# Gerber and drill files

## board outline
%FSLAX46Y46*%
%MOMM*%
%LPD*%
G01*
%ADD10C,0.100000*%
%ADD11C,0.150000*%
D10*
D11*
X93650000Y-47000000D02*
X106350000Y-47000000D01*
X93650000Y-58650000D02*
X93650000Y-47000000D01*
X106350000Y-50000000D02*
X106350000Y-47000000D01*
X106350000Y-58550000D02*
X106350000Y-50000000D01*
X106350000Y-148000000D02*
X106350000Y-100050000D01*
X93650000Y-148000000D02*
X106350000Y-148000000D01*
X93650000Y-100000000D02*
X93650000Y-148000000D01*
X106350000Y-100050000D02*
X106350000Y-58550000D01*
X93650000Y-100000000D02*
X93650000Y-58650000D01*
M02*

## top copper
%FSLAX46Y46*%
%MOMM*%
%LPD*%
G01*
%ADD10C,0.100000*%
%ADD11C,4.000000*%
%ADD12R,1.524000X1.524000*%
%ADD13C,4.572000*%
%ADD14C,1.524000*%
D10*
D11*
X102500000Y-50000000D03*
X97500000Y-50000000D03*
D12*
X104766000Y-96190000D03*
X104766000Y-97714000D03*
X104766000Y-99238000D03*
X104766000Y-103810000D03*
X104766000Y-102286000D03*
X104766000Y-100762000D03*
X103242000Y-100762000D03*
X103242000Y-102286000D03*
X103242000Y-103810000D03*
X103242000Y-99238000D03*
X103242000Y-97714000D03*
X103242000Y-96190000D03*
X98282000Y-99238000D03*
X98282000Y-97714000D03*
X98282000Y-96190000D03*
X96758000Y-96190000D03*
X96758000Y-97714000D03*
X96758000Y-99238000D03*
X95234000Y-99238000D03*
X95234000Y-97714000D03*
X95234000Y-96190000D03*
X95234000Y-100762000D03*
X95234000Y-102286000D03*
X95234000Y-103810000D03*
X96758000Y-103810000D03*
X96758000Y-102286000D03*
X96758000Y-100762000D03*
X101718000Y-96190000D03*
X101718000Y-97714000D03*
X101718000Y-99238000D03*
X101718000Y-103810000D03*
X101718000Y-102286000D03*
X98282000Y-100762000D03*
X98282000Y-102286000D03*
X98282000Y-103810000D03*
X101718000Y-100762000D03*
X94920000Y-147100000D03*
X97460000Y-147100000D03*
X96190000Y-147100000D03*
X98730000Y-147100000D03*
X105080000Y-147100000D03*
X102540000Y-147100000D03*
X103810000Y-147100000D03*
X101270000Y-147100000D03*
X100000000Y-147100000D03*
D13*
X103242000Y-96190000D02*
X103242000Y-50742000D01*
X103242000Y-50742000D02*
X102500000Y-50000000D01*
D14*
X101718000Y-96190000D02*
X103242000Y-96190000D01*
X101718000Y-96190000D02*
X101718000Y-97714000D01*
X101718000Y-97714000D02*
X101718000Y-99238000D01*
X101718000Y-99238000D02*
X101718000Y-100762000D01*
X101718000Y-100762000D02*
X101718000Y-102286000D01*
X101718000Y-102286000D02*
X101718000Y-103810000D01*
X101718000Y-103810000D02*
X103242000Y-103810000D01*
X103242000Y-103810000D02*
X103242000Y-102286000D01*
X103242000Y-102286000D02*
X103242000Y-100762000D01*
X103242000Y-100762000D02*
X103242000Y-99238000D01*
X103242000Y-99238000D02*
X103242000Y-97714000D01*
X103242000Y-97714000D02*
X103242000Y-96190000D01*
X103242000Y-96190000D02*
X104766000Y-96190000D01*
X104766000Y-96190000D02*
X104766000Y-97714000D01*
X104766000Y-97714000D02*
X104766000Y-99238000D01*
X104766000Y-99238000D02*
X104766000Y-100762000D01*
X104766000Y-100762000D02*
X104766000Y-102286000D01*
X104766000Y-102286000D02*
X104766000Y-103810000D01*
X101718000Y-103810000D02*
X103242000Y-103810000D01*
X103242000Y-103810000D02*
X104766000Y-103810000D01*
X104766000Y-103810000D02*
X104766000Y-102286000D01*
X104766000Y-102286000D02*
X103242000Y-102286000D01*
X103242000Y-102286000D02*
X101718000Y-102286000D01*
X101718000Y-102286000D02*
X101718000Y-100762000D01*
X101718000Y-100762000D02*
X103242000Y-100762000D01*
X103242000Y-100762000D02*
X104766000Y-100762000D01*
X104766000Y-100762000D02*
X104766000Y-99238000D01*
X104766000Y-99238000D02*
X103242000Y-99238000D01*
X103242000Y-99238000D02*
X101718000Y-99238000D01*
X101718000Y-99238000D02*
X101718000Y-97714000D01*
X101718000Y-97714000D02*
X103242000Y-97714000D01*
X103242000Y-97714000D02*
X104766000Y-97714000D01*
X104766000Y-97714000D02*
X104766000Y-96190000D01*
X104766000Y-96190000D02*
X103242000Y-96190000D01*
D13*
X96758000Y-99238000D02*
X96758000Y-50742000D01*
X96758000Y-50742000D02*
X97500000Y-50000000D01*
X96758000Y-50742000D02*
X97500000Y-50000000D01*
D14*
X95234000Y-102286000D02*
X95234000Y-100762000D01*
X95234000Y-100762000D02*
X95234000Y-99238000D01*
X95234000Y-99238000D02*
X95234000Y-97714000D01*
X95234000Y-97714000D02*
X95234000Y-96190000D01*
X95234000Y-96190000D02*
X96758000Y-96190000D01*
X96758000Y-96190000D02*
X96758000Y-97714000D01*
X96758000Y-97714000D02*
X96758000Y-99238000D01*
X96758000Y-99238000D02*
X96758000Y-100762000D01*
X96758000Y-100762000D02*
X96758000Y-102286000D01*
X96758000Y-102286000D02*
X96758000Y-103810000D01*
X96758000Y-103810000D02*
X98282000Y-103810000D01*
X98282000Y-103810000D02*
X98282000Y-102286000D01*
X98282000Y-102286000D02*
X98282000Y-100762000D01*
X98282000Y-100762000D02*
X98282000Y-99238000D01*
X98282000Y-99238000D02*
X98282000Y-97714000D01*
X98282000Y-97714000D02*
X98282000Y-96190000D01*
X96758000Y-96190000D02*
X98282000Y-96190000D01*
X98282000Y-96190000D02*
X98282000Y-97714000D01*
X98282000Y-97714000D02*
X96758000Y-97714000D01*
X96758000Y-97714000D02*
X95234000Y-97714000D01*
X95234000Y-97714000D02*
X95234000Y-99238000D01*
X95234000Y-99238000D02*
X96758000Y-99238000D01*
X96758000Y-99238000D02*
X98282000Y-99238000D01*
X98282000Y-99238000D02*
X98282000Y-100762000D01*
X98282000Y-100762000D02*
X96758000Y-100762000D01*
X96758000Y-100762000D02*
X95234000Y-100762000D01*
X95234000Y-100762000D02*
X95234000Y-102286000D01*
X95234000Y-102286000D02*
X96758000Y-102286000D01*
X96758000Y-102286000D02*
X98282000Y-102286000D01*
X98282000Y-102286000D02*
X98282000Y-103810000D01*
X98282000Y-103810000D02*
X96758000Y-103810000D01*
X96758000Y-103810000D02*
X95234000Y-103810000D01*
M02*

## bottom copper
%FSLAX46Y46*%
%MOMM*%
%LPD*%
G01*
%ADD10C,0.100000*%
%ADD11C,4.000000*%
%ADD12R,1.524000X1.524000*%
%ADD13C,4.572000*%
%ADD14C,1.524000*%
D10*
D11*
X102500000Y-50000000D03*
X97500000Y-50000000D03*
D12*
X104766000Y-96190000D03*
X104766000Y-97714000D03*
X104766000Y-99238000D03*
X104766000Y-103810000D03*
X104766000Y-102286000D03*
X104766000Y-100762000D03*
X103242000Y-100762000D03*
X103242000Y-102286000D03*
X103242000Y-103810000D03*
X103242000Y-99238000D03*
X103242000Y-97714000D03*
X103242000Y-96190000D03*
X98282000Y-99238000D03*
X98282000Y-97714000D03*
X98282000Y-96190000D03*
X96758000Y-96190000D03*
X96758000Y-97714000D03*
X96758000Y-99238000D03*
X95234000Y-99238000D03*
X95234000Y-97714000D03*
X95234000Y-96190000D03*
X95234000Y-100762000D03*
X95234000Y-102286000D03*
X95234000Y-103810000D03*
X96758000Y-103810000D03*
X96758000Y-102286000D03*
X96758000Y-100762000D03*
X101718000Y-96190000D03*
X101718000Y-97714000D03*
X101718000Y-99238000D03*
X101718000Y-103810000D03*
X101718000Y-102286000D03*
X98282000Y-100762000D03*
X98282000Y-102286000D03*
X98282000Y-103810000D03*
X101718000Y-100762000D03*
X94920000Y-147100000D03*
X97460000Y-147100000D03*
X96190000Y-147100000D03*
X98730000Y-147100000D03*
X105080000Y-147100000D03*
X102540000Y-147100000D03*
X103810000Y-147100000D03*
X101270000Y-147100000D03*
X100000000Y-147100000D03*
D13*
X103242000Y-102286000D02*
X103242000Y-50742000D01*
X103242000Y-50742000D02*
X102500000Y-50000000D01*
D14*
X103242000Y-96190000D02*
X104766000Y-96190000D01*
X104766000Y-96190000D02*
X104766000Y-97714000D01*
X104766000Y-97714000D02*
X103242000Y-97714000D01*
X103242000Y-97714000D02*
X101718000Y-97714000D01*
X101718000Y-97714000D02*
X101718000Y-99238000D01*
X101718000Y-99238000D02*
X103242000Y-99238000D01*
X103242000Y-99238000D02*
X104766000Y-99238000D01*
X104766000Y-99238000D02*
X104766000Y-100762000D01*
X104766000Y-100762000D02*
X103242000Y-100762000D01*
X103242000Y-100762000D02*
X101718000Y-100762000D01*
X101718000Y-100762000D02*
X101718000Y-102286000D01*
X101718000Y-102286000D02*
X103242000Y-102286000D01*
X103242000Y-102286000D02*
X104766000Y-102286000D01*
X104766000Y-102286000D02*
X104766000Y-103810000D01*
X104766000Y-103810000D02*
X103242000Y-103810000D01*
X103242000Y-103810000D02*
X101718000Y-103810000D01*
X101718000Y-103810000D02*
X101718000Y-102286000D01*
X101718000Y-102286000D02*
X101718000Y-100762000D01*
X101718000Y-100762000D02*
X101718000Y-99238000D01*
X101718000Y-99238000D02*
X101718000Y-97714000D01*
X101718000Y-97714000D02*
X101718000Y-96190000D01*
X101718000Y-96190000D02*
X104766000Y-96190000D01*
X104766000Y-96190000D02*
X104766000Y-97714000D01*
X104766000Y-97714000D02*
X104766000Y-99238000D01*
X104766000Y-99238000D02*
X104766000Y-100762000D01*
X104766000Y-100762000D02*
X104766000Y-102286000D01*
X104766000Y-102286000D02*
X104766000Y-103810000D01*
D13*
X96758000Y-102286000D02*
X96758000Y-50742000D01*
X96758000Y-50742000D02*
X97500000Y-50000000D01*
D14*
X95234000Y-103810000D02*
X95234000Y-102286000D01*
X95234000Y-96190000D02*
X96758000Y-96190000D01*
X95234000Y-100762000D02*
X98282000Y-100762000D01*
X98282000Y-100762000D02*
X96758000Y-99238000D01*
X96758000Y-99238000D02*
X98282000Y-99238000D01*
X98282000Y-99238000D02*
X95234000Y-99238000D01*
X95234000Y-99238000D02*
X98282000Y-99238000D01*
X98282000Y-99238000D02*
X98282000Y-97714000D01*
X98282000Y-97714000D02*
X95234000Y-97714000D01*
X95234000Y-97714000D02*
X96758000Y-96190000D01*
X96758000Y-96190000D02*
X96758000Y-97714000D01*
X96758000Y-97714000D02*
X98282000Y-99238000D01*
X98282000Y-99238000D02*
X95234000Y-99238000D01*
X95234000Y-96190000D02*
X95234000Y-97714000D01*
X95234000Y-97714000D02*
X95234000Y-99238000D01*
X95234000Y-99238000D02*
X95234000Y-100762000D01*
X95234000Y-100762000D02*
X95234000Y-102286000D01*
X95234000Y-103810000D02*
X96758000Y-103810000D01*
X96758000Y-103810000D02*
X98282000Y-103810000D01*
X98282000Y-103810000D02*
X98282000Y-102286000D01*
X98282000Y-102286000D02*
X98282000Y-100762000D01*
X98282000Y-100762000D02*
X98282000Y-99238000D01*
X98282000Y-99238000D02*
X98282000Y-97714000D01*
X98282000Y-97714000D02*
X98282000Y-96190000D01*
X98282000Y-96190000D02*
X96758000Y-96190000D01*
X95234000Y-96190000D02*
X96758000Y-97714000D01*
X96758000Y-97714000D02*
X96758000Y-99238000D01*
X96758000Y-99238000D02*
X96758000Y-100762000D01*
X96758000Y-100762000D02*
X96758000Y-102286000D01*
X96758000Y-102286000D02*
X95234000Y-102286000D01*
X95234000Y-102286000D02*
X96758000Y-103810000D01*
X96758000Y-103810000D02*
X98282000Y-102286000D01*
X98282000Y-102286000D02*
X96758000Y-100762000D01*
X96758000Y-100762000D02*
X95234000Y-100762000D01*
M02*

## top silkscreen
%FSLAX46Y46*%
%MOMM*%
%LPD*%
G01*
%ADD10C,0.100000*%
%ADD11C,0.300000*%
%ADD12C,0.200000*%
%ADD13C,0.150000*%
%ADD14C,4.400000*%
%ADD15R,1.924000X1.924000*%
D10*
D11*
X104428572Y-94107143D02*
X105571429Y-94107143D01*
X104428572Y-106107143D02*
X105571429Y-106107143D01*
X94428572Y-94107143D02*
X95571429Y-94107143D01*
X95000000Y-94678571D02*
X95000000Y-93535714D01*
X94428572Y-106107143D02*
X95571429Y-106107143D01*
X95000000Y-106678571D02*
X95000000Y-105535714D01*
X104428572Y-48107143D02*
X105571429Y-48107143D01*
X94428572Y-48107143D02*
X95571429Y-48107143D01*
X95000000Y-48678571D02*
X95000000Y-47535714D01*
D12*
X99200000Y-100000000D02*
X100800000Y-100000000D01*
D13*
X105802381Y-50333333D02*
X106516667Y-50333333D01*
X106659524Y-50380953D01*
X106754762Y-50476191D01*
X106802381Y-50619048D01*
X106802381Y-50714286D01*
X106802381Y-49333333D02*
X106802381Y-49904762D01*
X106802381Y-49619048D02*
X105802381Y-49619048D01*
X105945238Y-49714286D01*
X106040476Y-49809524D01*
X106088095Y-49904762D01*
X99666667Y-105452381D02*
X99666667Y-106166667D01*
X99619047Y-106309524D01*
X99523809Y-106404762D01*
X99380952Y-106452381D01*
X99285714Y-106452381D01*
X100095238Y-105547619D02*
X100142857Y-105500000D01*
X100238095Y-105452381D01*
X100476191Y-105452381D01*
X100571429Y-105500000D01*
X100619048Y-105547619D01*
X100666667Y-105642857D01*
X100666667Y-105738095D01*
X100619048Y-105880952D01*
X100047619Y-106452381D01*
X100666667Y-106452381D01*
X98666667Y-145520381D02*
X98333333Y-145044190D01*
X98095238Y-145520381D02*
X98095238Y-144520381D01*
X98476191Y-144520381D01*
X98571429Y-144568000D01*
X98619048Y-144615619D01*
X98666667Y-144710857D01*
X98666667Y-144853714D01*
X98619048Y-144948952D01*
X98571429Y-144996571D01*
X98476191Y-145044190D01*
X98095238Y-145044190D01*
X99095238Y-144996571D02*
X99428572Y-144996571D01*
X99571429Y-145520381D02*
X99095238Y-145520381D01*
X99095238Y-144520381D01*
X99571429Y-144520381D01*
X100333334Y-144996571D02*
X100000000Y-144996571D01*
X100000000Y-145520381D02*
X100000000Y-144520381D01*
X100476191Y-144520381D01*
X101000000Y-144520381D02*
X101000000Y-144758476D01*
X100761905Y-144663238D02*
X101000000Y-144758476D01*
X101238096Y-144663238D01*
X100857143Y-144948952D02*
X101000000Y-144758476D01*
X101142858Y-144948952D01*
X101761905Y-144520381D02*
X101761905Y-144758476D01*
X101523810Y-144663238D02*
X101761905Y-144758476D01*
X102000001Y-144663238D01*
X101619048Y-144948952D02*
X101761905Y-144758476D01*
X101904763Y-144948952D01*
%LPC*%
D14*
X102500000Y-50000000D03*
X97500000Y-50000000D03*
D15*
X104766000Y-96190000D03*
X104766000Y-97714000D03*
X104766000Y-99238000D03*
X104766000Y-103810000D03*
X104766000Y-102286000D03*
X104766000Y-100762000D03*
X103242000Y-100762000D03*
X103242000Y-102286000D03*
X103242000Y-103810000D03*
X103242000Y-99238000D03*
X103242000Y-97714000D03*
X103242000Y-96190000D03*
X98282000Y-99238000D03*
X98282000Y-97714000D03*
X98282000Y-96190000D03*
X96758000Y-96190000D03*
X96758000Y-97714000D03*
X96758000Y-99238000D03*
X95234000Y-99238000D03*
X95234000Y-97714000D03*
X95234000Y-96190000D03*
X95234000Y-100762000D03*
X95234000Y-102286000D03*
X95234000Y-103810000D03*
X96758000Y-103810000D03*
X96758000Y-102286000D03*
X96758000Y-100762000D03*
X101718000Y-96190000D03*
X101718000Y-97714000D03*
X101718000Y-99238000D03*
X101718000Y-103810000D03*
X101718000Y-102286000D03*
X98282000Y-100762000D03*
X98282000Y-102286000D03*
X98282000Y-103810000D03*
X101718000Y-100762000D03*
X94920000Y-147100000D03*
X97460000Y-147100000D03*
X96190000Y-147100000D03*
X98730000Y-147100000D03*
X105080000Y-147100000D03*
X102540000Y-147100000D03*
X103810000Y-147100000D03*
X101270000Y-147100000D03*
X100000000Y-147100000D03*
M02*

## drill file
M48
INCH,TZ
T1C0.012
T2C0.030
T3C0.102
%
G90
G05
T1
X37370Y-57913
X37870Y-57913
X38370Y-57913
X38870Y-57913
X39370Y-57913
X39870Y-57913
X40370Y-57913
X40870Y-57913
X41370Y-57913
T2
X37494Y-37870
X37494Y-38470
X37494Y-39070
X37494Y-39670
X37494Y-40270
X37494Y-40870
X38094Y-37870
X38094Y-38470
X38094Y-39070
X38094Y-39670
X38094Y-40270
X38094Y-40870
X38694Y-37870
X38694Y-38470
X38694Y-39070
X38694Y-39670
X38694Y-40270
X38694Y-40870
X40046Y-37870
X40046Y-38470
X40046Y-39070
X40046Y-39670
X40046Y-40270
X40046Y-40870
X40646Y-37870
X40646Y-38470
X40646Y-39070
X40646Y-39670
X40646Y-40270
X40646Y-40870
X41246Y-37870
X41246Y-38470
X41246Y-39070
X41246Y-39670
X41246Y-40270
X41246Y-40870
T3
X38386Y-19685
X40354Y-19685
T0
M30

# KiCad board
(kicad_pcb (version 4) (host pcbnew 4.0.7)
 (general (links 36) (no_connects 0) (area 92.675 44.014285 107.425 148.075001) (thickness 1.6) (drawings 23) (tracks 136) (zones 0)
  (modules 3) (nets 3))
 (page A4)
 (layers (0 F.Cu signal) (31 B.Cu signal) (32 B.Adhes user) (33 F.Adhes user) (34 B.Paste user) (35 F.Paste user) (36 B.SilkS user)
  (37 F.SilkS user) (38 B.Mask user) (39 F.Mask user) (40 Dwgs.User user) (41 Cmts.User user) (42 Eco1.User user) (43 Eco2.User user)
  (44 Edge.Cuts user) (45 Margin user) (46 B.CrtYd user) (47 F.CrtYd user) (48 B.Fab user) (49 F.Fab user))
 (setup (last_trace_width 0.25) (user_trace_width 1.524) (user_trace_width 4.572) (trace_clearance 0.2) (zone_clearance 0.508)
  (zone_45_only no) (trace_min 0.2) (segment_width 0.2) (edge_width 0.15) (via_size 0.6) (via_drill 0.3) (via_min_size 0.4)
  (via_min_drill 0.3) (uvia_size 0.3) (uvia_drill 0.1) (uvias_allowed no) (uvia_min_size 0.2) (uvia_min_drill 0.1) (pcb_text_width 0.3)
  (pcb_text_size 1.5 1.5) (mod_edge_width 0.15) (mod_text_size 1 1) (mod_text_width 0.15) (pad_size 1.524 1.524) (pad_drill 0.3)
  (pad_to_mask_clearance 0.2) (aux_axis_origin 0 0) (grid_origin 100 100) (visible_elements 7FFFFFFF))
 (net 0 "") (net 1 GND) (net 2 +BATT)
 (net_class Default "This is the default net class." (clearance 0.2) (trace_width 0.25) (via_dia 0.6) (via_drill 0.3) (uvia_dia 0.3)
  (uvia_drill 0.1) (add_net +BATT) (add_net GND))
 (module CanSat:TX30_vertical (layer F.Cu) (at 100 50 90)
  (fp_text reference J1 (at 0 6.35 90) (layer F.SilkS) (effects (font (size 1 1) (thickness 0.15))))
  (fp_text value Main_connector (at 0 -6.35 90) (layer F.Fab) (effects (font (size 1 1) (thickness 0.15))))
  (pad 2 thru_hole circle (at 0 2.5 90) (size 4 4) (drill 2.6) (layers *.Cu *.Mask) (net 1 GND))
  (pad 1 thru_hole circle (at 0 -2.5 90) (size 4 4) (drill 2.6) (layers *.Cu *.Mask) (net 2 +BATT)))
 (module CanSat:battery (layer F.Cu) (at 100 100)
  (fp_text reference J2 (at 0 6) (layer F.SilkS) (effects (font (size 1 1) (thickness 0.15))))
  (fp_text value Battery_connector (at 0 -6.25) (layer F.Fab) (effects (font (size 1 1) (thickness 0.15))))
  (pad 2 thru_hole rect (at 4.766 -3.81) (size 1.524 1.524) (drill 0.762) (layers *.Cu *.Mask) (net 1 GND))
  (pad 2 thru_hole rect (at 4.766 -2.286) (size 1.524 1.524) (drill 0.762) (layers *.Cu *.Mask) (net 1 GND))
  (pad 2 thru_hole rect (at 4.766 -0.762) (size 1.524 1.524) (drill 0.762) (layers *.Cu *.Mask) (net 1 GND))
  (pad 2 thru_hole rect (at 4.766 3.81) (size 1.524 1.524) (drill 0.762) (layers *.Cu *.Mask) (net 1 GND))
  (pad 2 thru_hole rect (at 4.766 2.286) (size 1.524 1.524) (drill 0.762) (layers *.Cu *.Mask) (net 1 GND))
  (pad 2 thru_hole rect (at 4.766 0.762) (size 1.524 1.524) (drill 0.762) (layers *.Cu *.Mask) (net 1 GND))
  (pad 2 thru_hole rect (at 3.242 0.762) (size 1.524 1.524) (drill 0.762) (layers *.Cu *.Mask) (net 1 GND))
  (pad 2 thru_hole rect (at 3.242 2.286) (size 1.524 1.524) (drill 0.762) (layers *.Cu *.Mask) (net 1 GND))
  (pad 2 thru_hole rect (at 3.242 3.81) (size 1.524 1.524) (drill 0.762) (layers *.Cu *.Mask) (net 1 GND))
  (pad 2 thru_hole rect (at 3.242 -0.762) (size 1.524 1.524) (drill 0.762) (layers *.Cu *.Mask) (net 1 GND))
  (pad 2 thru_hole rect (at 3.242 -2.286) (size 1.524 1.524) (drill 0.762) (layers *.Cu *.Mask) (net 1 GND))
  (pad 2 thru_hole rect (at 3.242 -3.81) (size 1.524 1.524) (drill 0.762) (layers *.Cu *.Mask) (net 1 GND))
  (pad 1 thru_hole rect (at -1.718 -0.762) (size 1.524 1.524) (drill 0.762) (layers *.Cu *.Mask) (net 2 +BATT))
  (pad 1 thru_hole rect (at -1.718 -2.286) (size 1.524 1.524) (drill 0.762) (layers *.Cu *.Mask) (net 2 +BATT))
  (pad 1 thru_hole rect (at -1.718 -3.81) (size 1.524 1.524) (drill 0.762) (layers *.Cu *.Mask) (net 2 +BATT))
  (pad 1 thru_hole rect (at -3.242 -3.81) (size 1.524 1.524) (drill 0.762) (layers *.Cu *.Mask) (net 2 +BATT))
  (pad 1 thru_hole rect (at -3.242 -2.286) (size 1.524 1.524) (drill 0.762) (layers *.Cu *.Mask) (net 2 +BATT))
  (pad 1 thru_hole rect (at -3.242 -0.762) (size 1.524 1.524) (drill 0.762) (layers *.Cu *.Mask) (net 2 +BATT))
  (pad 1 thru_hole rect (at -4.766 -0.762) (size 1.524 1.524) (drill 0.762) (layers *.Cu *.Mask) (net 2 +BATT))
  (pad 1 thru_hole rect (at -4.766 -2.286) (size 1.524 1.524) (drill 0.762) (layers *.Cu *.Mask) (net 2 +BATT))
  (pad 1 thru_hole rect (at -4.766 -3.81) (size 1.524 1.524) (drill 0.762) (layers *.Cu *.Mask) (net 2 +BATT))
  (pad 1 thru_hole rect (at -4.766 0.762) (size 1.524 1.524) (drill 0.762) (layers *.Cu *.Mask) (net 2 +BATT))
  (pad 1 thru_hole rect (at -4.766 2.286) (size 1.524 1.524) (drill 0.762) (layers *.Cu *.Mask) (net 2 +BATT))
  (pad 1 thru_hole rect (at -4.766 3.81) (size 1.524 1.524) (drill 0.762) (layers *.Cu *.Mask) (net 2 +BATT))
  (pad 1 thru_hole rect (at -3.242 3.81) (size 1.524 1.524) (drill 0.762) (layers *.Cu *.Mask) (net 2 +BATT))
  (pad 1 thru_hole rect (at -3.242 2.286) (size 1.524 1.524) (drill 0.762) (layers *.Cu *.Mask) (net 2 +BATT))
  (pad 1 thru_hole rect (at -3.242 0.762) (size 1.524 1.524) (drill 0.762) (layers *.Cu *.Mask) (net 2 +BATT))
  (pad 2 thru_hole rect (at 1.718 -3.81) (size 1.524 1.524) (drill 0.762) (layers *.Cu *.Mask) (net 1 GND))
  (pad 2 thru_hole rect (at 1.718 -2.286) (size 1.524 1.524) (drill 0.762) (layers *.Cu *.Mask) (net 1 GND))
  (pad 2 thru_hole rect (at 1.718 -0.762) (size 1.524 1.524) (drill 0.762) (layers *.Cu *.Mask) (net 1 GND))
  (pad 2 thru_hole rect (at 1.718 3.81) (size 1.524 1.524) (drill 0.762) (layers *.Cu *.Mask) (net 1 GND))
  (pad 2 thru_hole rect (at 1.718 2.286) (size 1.524 1.524) (drill 0.762) (layers *.Cu *.Mask) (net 1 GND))
  (pad 1 thru_hole rect (at -1.718 0.762) (size 1.524 1.524) (drill 0.762) (layers *.Cu *.Mask) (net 2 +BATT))
  (pad 1 thru_hole rect (at -1.718 2.286) (size 1.524 1.524) (drill 0.762) (layers *.Cu *.Mask) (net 2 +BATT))
  (pad 1 thru_hole rect (at -1.718 3.81) (size 1.524 1.524) (drill 0.762) (layers *.Cu *.Mask) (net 2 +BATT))
  (pad 2 thru_hole rect (at 1.718 0.762) (size 1.524 1.524) (drill 0.762) (layers *.Cu *.Mask) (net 1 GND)))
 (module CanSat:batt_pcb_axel (layer F.Cu) (at 100 147.1)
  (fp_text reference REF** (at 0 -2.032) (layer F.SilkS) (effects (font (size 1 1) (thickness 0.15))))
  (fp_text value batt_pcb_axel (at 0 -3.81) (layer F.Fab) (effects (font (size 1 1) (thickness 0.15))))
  (pad "" thru_hole rect (at -5.08 0) (size 1.524 1.524) (drill 0.3) (layers *.Cu *.Mask))
  (pad "" thru_hole rect (at -2.54 0) (size 1.524 1.524) (drill 0.3) (layers *.Cu *.Mask))
  (pad "" thru_hole rect (at -3.81 0) (size 1.524 1.524) (drill 0.3) (layers *.Cu *.Mask))
  (pad "" thru_hole rect (at -1.27 0) (size 1.524 1.524) (drill 0.3) (layers *.Cu *.Mask))
  (pad "" thru_hole rect (at 5.08 0) (size 1.524 1.524) (drill 0.3) (layers *.Cu *.Mask))
  (pad "" thru_hole rect (at 2.54 0) (size 1.524 1.524) (drill 0.3) (layers *.Cu *.Mask))
  (pad "" thru_hole rect (at 3.81 0) (size 1.524 1.524) (drill 0.3) (layers *.Cu *.Mask))
  (pad "" thru_hole rect (at 1.27 0) (size 1.524 1.524) (drill 0.3) (layers *.Cu *.Mask))
  (pad "" thru_hole rect (at 0 0) (size 1.524 1.524) (drill 0.3) (layers *.Cu *.Mask)))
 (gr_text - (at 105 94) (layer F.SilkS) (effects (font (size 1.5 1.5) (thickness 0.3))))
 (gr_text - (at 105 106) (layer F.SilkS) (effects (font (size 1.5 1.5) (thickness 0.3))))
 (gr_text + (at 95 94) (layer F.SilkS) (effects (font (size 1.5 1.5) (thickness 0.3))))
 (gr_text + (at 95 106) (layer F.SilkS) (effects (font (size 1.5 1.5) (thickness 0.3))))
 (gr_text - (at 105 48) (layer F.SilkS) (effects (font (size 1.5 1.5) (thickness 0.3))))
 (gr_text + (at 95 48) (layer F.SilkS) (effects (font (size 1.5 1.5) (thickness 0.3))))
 (gr_line (start 93.65 47) (end 106.35 47) (angle 90) (layer Edge.Cuts) (width 0.15))
 (gr_line (start 93.65 58.65) (end 93.65 47) (angle 90) (layer Edge.Cuts) (width 0.15))
 (gr_line (start 106.35 50) (end 106.35 47) (angle 90) (layer Edge.Cuts) (width 0.15))
 (gr_line (start 106.35 58.55) (end 106.35 50) (angle 90) (layer Edge.Cuts) (width 0.15))
 (gr_line (start 106.35 148) (end 106.35 100.05) (angle 90) (layer Edge.Cuts) (width 0.15))
 (gr_line (start 93.65 148) (end 106.35 148) (angle 90) (layer Edge.Cuts) (width 0.15))
 (gr_line (start 93.65 100) (end 93.65 148) (angle 90) (layer Edge.Cuts) (width 0.15))
 (gr_line (start 106.35 100.05) (end 106.35 58.55) (angle 90) (layer Edge.Cuts) (width 0.15))
 (gr_line (start 93.65 100) (end 93.65 58.65) (angle 90) (layer Edge.Cuts) (width 0.15))
 (gr_line (start 99.2 100) (end 100.8 100) (angle 90) (layer F.SilkS) (width 0.2))
 (segment (start 103.242 102.286) (end 103.242 50.742) (width 4.572) (layer B.Cu) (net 1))
 (segment (start 103.242 50.742) (end 102.5 50) (width 4.572) (layer B.Cu) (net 1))
 (segment (start 103.242 96.19) (end 103.242 50.742) (width 4.572) (layer F.Cu) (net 1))
 (segment (start 103.242 50.742) (end 102.5 50) (width 4.572) (layer F.Cu) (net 1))
 (segment (start 101.718 96.19) (end 103.242 96.19) (width 1.524) (layer F.Cu) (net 1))
 (segment (start 103.242 96.19) (end 104.766 96.19) (width 1.524) (layer B.Cu) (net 1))
 (segment (start 104.766 96.19) (end 104.766 97.714) (width 1.524) (layer B.Cu) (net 1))
 (segment (start 104.766 97.714) (end 103.242 97.714) (width 1.524) (layer B.Cu) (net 1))
 (segment (start 103.242 97.714) (end 101.718 97.714) (width 1.524) (layer B.Cu) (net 1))
 (segment (start 101.718 97.714) (end 101.718 99.238) (width 1.524) (layer B.Cu) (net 1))
 (segment (start 101.718 99.238) (end 103.242 99.238) (width 1.524) (layer B.Cu) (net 1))
 (segment (start 103.242 99.238) (end 104.766 99.238) (width 1.524) (layer B.Cu) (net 1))
 (segment (start 104.766 99.238) (end 104.766 100.762) (width 1.524) (layer B.Cu) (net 1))
 (segment (start 104.766 100.762) (end 103.242 100.762) (width 1.524) (layer B.Cu) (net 1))
 (segment (start 103.242 100.762) (end 101.718 100.762) (width 1.524) (layer B.Cu) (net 1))
 (segment (start 101.718 100.762) (end 101.718 102.286) (width 1.524) (layer B.Cu) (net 1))
 (segment (start 101.718 102.286) (end 103.242 102.286) (width 1.524) (layer B.Cu) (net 1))
 (segment (start 103.242 102.286) (end 104.766 102.286) (width 1.524) (layer B.Cu) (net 1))
 (segment (start 104.766 102.286) (end 104.766 103.81) (width 1.524) (layer B.Cu) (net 1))
 (segment (start 104.766 103.81) (end 103.242 103.81) (width 1.524) (layer B.Cu) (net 1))
 (segment (start 103.242 103.81) (end 101.718 103.81) (width 1.524) (layer B.Cu) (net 1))
 (segment (start 101.718 103.81) (end 101.718 102.286) (width 1.524) (layer B.Cu) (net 1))
 (segment (start 101.718 102.286) (end 101.718 100.762) (width 1.524) (layer B.Cu) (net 1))
 (segment (start 101.718 100.762) (end 101.718 99.238) (width 1.524) (layer B.Cu) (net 1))
 (segment (start 101.718 99.238) (end 101.718 97.714) (width 1.524) (layer B.Cu) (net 1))
 (segment (start 101.718 97.714) (end 101.718 96.19) (width 1.524) (layer B.Cu) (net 1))
 (segment (start 101.718 96.19) (end 104.766 96.19) (width 1.524) (layer B.Cu) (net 1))
 (segment (start 104.766 96.19) (end 104.766 97.714) (width 1.524) (layer B.Cu) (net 1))
 (segment (start 104.766 97.714) (end 104.766 99.238) (width 1.524) (layer B.Cu) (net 1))
 (segment (start 104.766 99.238) (end 104.766 100.762) (width 1.524) (layer B.Cu) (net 1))
 (segment (start 104.766 100.762) (end 104.766 102.286) (width 1.524) (layer B.Cu) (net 1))
 (segment (start 104.766 102.286) (end 104.766 103.81) (width 1.524) (layer B.Cu) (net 1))
 (segment (start 101.718 96.19) (end 101.718 97.714) (width 1.524) (layer F.Cu) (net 1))
 (segment (start 101.718 97.714) (end 101.718 99.238) (width 1.524) (layer F.Cu) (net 1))
 (segment (start 101.718 99.238) (end 101.718 100.762) (width 1.524) (layer F.Cu) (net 1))
 (segment (start 101.718 100.762) (end 101.718 102.286) (width 1.524) (layer F.Cu) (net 1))
 (segment (start 101.718 102.286) (end 101.718 103.81) (width 1.524) (layer F.Cu) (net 1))
 (segment (start 101.718 103.81) (end 103.242 103.81) (width 1.524) (layer F.Cu) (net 1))
 (segment (start 103.242 103.81) (end 103.242 102.286) (width 1.524) (layer F.Cu) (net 1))
 (segment (start 103.242 102.286) (end 103.242 100.762) (width 1.524) (layer F.Cu) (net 1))
 (segment (start 103.242 100.762) (end 103.242 99.238) (width 1.524) (layer F.Cu) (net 1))
 (segment (start 103.242 99.238) (end 103.242 97.714) (width 1.524) (layer F.Cu) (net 1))
 (segment (start 103.242 97.714) (end 103.242 96.19) (width 1.524) (layer F.Cu) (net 1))
 (segment (start 103.242 96.19) (end 104.766 96.19) (width 1.524) (layer F.Cu) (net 1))
 (segment (start 104.766 96.19) (end 104.766 97.714) (width 1.524) (layer F.Cu) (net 1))
 (segment (start 104.766 97.714) (end 104.766 99.238) (width 1.524) (layer F.Cu) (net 1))
 (segment (start 104.766 99.238) (end 104.766 100.762) (width 1.524) (layer F.Cu) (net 1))
 (segment (start 104.766 100.762) (end 104.766 102.286) (width 1.524) (layer F.Cu) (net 1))
 (segment (start 104.766 102.286) (end 104.766 103.81) (width 1.524) (layer F.Cu) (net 1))
 (segment (start 101.718 103.81) (end 103.242 103.81) (width 1.524) (layer F.Cu) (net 1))
 (segment (start 103.242 103.81) (end 104.766 103.81) (width 1.524) (layer F.Cu) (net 1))
 (segment (start 104.766 103.81) (end 104.766 102.286) (width 1.524) (layer F.Cu) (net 1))
 (segment (start 104.766 102.286) (end 103.242 102.286) (width 1.524) (layer F.Cu) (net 1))
 (segment (start 103.242 102.286) (end 101.718 102.286) (width 1.524) (layer F.Cu) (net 1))
 (segment (start 101.718 102.286) (end 101.718 100.762) (width 1.524) (layer F.Cu) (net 1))
 (segment (start 101.718 100.762) (end 103.242 100.762) (width 1.524) (layer F.Cu) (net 1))
 (segment (start 103.242 100.762) (end 104.766 100.762) (width 1.524) (layer F.Cu) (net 1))
 (segment (start 104.766 100.762) (end 104.766 99.238) (width 1.524) (layer F.Cu) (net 1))
 (segment (start 104.766 99.238) (end 103.242 99.238) (width 1.524) (layer F.Cu) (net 1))
 (segment (start 103.242 99.238) (end 101.718 99.238) (width 1.524) (layer F.Cu) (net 1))
 (segment (start 101.718 99.238) (end 101.718 97.714) (width 1.524) (layer F.Cu) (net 1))
 (segment (start 101.718 97.714) (end 103.242 97.714) (width 1.524) (layer F.Cu) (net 1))
 (segment (start 103.242 97.714) (end 104.766 97.714) (width 1.524) (layer F.Cu) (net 1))
 (segment (start 104.766 97.714) (end 104.766 96.19) (width 1.524) (layer F.Cu) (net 1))
 (segment (start 104.766 96.19) (end 103.242 96.19) (width 1.524) (layer F.Cu) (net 1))
 (segment (start 96.758 99.238) (end 96.758 50.742) (width 4.572) (layer F.Cu) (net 2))
 (segment (start 96.758 50.742) (end 97.5 50) (width 4.572) (layer F.Cu) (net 2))
 (segment (start 96.758 102.286) (end 96.758 50.742) (width 4.572) (layer B.Cu) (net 2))
 (segment (start 96.758 50.742) (end 97.5 50) (width 4.572) (layer B.Cu) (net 2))
 (segment (start 96.758 50.742) (end 97.5 50) (width 4.572) (layer F.Cu) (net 2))
 (segment (start 95.234 103.81) (end 95.234 102.286) (width 1.524) (layer B.Cu) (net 2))
 (segment (start 95.234 102.286) (end 95.234 100.762) (width 1.524) (layer F.Cu) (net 2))
 (segment (start 95.234 100.762) (end 95.234 99.238) (width 1.524) (layer F.Cu) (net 2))
 (segment (start 95.234 99.238) (end 95.234 97.714) (width 1.524) (layer F.Cu) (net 2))
 (segment (start 95.234 97.714) (end 95.234 96.19) (width 1.524) (layer F.Cu) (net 2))
 (segment (start 95.234 96.19) (end 96.758 96.19) (width 1.524) (layer F.Cu) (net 2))
 (segment (start 96.758 96.19) (end 96.758 97.714) (width 1.524) (layer F.Cu) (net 2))
 (segment (start 96.758 97.714) (end 96.758 99.238) (width 1.524) (layer F.Cu) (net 2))
 (segment (start 96.758 99.238) (end 96.758 100.762) (width 1.524) (layer F.Cu) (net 2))
 (segment (start 96.758 100.762) (end 96.758 102.286) (width 1.524) (layer F.Cu) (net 2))
 (segment (start 96.758 102.286) (end 96.758 103.81) (width 1.524) (layer F.Cu) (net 2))
 (segment (start 96.758 103.81) (end 98.282 103.81) (width 1.524) (layer F.Cu) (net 2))
 (segment (start 98.282 103.81) (end 98.282 102.286) (width 1.524) (layer F.Cu) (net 2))
 (segment (start 98.282 102.286) (end 98.282 100.762) (width 1.524) (layer F.Cu) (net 2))
 (segment (start 98.282 100.762) (end 98.282 99.238) (width 1.524) (layer F.Cu) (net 2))
 (segment (start 98.282 99.238) (end 98.282 97.714) (width 1.524) (layer F.Cu) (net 2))
 (segment (start 98.282 97.714) (end 98.282 96.19) (width 1.524) (layer F.Cu) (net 2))
 (segment (start 95.234 96.19) (end 96.758 96.19) (width 1.524) (layer B.Cu) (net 2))
 (segment (start 96.758 96.19) (end 98.282 96.19) (width 1.524) (layer F.Cu) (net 2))
 (segment (start 98.282 96.19) (end 98.282 97.714) (width 1.524) (layer F.Cu) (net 2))
 (segment (start 98.282 97.714) (end 96.758 97.714) (width 1.524) (layer F.Cu) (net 2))
 (segment (start 96.758 97.714) (end 95.234 97.714) (width 1.524) (layer F.Cu) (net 2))
 (segment (start 95.234 97.714) (end 95.234 99.238) (width 1.524) (layer F.Cu) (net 2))
 (segment (start 95.234 99.238) (end 96.758 99.238) (width 1.524) (layer F.Cu) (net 2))
 (segment (start 96.758 99.238) (end 98.282 99.238) (width 1.524) (layer F.Cu) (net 2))
 (segment (start 98.282 99.238) (end 98.282 100.762) (width 1.524) (layer F.Cu) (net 2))
 (segment (start 98.282 100.762) (end 96.758 100.762) (width 1.524) (layer F.Cu) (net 2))
 (segment (start 96.758 100.762) (end 95.234 100.762) (width 1.524) (layer F.Cu) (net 2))
 (segment (start 95.234 100.762) (end 95.234 102.286) (width 1.524) (layer F.Cu) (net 2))
 (segment (start 95.234 102.286) (end 96.758 102.286) (width 1.524) (layer F.Cu) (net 2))
 (segment (start 96.758 102.286) (end 98.282 102.286) (width 1.524) (layer F.Cu) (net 2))
 (segment (start 98.282 102.286) (end 98.282 103.81) (width 1.524) (layer F.Cu) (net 2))
 (segment (start 98.282 103.81) (end 96.758 103.81) (width 1.524) (layer F.Cu) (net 2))
 (segment (start 96.758 103.81) (end 95.234 103.81) (width 1.524) (layer F.Cu) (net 2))
 (segment (start 95.234 100.762) (end 98.282 100.762) (width 1.524) (layer B.Cu) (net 2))
 (segment (start 98.282 100.762) (end 96.758 99.238) (width 1.524) (layer B.Cu) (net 2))
 (segment (start 96.758 99.238) (end 98.282 99.238) (width 1.524) (layer B.Cu) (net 2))
 (segment (start 98.282 99.238) (end 95.234 99.238) (width 1.524) (layer B.Cu) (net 2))
 (segment (start 95.234 99.238) (end 98.282 99.238) (width 1.524) (layer B.Cu) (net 2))
 (segment (start 98.282 99.238) (end 98.282 97.714) (width 1.524) (layer B.Cu) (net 2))
 (segment (start 98.282 97.714) (end 95.234 97.714) (width 1.524) (layer B.Cu) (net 2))
 (segment (start 95.234 97.714) (end 96.758 96.19) (width 1.524) (layer B.Cu) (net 2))
 (segment (start 96.758 96.19) (end 96.758 97.714) (width 1.524) (layer B.Cu) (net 2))
 (segment (start 96.758 97.714) (end 98.282 99.238) (width 1.524) (layer B.Cu) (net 2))
 (segment (start 98.282 99.238) (end 95.234 99.238) (width 1.524) (layer B.Cu) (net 2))
 (segment (start 95.234 96.19) (end 95.234 97.714) (width 1.524) (layer B.Cu) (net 2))
 (segment (start 95.234 97.714) (end 95.234 99.238) (width 1.524) (layer B.Cu) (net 2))
 (segment (start 95.234 99.238) (end 95.234 100.762) (width 1.524) (layer B.Cu) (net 2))
 (segment (start 95.234 100.762) (end 95.234 102.286) (width 1.524) (layer B.Cu) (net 2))
 (segment (start 95.234 103.81) (end 96.758 103.81) (width 1.524) (layer B.Cu) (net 2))
 (segment (start 96.758 103.81) (end 98.282 103.81) (width 1.524) (layer B.Cu) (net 2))
 (segment (start 98.282 103.81) (end 98.282 102.286) (width 1.524) (layer B.Cu) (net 2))
 (segment (start 98.282 102.286) (end 98.282 100.762) (width 1.524) (layer B.Cu) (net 2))
 (segment (start 98.282 100.762) (end 98.282 99.238) (width 1.524) (layer B.Cu) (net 2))
 (segment (start 98.282 99.238) (end 98.282 97.714) (width 1.524) (layer B.Cu) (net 2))
 (segment (start 98.282 97.714) (end 98.282 96.19) (width 1.524) (layer B.Cu) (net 2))
 (segment (start 98.282 96.19) (end 96.758 96.19) (width 1.524) (layer B.Cu) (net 2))
 (segment (start 95.234 96.19) (end 96.758 97.714) (width 1.524) (layer B.Cu) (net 2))
 (segment (start 96.758 97.714) (end 96.758 99.238) (width 1.524) (layer B.Cu) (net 2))
 (segment (start 96.758 99.238) (end 96.758 100.762) (width 1.524) (layer B.Cu) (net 2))
 (segment (start 96.758 100.762) (end 96.758 102.286) (width 1.524) (layer B.Cu) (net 2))
 (segment (start 96.758 102.286) (end 95.234 102.286) (width 1.524) (layer B.Cu) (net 2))
 (segment (start 95.234 102.286) (end 96.758 103.81) (width 1.524) (layer B.Cu) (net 2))
 (segment (start 96.758 103.81) (end 98.282 102.286) (width 1.524) (layer B.Cu) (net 2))
 (segment (start 98.282 102.286) (end 96.758 100.762) (width 1.524) (layer B.Cu) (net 2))
 (segment (start 96.758 100.762) (end 95.234 100.762) (width 1.524) (layer B.Cu) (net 2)))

